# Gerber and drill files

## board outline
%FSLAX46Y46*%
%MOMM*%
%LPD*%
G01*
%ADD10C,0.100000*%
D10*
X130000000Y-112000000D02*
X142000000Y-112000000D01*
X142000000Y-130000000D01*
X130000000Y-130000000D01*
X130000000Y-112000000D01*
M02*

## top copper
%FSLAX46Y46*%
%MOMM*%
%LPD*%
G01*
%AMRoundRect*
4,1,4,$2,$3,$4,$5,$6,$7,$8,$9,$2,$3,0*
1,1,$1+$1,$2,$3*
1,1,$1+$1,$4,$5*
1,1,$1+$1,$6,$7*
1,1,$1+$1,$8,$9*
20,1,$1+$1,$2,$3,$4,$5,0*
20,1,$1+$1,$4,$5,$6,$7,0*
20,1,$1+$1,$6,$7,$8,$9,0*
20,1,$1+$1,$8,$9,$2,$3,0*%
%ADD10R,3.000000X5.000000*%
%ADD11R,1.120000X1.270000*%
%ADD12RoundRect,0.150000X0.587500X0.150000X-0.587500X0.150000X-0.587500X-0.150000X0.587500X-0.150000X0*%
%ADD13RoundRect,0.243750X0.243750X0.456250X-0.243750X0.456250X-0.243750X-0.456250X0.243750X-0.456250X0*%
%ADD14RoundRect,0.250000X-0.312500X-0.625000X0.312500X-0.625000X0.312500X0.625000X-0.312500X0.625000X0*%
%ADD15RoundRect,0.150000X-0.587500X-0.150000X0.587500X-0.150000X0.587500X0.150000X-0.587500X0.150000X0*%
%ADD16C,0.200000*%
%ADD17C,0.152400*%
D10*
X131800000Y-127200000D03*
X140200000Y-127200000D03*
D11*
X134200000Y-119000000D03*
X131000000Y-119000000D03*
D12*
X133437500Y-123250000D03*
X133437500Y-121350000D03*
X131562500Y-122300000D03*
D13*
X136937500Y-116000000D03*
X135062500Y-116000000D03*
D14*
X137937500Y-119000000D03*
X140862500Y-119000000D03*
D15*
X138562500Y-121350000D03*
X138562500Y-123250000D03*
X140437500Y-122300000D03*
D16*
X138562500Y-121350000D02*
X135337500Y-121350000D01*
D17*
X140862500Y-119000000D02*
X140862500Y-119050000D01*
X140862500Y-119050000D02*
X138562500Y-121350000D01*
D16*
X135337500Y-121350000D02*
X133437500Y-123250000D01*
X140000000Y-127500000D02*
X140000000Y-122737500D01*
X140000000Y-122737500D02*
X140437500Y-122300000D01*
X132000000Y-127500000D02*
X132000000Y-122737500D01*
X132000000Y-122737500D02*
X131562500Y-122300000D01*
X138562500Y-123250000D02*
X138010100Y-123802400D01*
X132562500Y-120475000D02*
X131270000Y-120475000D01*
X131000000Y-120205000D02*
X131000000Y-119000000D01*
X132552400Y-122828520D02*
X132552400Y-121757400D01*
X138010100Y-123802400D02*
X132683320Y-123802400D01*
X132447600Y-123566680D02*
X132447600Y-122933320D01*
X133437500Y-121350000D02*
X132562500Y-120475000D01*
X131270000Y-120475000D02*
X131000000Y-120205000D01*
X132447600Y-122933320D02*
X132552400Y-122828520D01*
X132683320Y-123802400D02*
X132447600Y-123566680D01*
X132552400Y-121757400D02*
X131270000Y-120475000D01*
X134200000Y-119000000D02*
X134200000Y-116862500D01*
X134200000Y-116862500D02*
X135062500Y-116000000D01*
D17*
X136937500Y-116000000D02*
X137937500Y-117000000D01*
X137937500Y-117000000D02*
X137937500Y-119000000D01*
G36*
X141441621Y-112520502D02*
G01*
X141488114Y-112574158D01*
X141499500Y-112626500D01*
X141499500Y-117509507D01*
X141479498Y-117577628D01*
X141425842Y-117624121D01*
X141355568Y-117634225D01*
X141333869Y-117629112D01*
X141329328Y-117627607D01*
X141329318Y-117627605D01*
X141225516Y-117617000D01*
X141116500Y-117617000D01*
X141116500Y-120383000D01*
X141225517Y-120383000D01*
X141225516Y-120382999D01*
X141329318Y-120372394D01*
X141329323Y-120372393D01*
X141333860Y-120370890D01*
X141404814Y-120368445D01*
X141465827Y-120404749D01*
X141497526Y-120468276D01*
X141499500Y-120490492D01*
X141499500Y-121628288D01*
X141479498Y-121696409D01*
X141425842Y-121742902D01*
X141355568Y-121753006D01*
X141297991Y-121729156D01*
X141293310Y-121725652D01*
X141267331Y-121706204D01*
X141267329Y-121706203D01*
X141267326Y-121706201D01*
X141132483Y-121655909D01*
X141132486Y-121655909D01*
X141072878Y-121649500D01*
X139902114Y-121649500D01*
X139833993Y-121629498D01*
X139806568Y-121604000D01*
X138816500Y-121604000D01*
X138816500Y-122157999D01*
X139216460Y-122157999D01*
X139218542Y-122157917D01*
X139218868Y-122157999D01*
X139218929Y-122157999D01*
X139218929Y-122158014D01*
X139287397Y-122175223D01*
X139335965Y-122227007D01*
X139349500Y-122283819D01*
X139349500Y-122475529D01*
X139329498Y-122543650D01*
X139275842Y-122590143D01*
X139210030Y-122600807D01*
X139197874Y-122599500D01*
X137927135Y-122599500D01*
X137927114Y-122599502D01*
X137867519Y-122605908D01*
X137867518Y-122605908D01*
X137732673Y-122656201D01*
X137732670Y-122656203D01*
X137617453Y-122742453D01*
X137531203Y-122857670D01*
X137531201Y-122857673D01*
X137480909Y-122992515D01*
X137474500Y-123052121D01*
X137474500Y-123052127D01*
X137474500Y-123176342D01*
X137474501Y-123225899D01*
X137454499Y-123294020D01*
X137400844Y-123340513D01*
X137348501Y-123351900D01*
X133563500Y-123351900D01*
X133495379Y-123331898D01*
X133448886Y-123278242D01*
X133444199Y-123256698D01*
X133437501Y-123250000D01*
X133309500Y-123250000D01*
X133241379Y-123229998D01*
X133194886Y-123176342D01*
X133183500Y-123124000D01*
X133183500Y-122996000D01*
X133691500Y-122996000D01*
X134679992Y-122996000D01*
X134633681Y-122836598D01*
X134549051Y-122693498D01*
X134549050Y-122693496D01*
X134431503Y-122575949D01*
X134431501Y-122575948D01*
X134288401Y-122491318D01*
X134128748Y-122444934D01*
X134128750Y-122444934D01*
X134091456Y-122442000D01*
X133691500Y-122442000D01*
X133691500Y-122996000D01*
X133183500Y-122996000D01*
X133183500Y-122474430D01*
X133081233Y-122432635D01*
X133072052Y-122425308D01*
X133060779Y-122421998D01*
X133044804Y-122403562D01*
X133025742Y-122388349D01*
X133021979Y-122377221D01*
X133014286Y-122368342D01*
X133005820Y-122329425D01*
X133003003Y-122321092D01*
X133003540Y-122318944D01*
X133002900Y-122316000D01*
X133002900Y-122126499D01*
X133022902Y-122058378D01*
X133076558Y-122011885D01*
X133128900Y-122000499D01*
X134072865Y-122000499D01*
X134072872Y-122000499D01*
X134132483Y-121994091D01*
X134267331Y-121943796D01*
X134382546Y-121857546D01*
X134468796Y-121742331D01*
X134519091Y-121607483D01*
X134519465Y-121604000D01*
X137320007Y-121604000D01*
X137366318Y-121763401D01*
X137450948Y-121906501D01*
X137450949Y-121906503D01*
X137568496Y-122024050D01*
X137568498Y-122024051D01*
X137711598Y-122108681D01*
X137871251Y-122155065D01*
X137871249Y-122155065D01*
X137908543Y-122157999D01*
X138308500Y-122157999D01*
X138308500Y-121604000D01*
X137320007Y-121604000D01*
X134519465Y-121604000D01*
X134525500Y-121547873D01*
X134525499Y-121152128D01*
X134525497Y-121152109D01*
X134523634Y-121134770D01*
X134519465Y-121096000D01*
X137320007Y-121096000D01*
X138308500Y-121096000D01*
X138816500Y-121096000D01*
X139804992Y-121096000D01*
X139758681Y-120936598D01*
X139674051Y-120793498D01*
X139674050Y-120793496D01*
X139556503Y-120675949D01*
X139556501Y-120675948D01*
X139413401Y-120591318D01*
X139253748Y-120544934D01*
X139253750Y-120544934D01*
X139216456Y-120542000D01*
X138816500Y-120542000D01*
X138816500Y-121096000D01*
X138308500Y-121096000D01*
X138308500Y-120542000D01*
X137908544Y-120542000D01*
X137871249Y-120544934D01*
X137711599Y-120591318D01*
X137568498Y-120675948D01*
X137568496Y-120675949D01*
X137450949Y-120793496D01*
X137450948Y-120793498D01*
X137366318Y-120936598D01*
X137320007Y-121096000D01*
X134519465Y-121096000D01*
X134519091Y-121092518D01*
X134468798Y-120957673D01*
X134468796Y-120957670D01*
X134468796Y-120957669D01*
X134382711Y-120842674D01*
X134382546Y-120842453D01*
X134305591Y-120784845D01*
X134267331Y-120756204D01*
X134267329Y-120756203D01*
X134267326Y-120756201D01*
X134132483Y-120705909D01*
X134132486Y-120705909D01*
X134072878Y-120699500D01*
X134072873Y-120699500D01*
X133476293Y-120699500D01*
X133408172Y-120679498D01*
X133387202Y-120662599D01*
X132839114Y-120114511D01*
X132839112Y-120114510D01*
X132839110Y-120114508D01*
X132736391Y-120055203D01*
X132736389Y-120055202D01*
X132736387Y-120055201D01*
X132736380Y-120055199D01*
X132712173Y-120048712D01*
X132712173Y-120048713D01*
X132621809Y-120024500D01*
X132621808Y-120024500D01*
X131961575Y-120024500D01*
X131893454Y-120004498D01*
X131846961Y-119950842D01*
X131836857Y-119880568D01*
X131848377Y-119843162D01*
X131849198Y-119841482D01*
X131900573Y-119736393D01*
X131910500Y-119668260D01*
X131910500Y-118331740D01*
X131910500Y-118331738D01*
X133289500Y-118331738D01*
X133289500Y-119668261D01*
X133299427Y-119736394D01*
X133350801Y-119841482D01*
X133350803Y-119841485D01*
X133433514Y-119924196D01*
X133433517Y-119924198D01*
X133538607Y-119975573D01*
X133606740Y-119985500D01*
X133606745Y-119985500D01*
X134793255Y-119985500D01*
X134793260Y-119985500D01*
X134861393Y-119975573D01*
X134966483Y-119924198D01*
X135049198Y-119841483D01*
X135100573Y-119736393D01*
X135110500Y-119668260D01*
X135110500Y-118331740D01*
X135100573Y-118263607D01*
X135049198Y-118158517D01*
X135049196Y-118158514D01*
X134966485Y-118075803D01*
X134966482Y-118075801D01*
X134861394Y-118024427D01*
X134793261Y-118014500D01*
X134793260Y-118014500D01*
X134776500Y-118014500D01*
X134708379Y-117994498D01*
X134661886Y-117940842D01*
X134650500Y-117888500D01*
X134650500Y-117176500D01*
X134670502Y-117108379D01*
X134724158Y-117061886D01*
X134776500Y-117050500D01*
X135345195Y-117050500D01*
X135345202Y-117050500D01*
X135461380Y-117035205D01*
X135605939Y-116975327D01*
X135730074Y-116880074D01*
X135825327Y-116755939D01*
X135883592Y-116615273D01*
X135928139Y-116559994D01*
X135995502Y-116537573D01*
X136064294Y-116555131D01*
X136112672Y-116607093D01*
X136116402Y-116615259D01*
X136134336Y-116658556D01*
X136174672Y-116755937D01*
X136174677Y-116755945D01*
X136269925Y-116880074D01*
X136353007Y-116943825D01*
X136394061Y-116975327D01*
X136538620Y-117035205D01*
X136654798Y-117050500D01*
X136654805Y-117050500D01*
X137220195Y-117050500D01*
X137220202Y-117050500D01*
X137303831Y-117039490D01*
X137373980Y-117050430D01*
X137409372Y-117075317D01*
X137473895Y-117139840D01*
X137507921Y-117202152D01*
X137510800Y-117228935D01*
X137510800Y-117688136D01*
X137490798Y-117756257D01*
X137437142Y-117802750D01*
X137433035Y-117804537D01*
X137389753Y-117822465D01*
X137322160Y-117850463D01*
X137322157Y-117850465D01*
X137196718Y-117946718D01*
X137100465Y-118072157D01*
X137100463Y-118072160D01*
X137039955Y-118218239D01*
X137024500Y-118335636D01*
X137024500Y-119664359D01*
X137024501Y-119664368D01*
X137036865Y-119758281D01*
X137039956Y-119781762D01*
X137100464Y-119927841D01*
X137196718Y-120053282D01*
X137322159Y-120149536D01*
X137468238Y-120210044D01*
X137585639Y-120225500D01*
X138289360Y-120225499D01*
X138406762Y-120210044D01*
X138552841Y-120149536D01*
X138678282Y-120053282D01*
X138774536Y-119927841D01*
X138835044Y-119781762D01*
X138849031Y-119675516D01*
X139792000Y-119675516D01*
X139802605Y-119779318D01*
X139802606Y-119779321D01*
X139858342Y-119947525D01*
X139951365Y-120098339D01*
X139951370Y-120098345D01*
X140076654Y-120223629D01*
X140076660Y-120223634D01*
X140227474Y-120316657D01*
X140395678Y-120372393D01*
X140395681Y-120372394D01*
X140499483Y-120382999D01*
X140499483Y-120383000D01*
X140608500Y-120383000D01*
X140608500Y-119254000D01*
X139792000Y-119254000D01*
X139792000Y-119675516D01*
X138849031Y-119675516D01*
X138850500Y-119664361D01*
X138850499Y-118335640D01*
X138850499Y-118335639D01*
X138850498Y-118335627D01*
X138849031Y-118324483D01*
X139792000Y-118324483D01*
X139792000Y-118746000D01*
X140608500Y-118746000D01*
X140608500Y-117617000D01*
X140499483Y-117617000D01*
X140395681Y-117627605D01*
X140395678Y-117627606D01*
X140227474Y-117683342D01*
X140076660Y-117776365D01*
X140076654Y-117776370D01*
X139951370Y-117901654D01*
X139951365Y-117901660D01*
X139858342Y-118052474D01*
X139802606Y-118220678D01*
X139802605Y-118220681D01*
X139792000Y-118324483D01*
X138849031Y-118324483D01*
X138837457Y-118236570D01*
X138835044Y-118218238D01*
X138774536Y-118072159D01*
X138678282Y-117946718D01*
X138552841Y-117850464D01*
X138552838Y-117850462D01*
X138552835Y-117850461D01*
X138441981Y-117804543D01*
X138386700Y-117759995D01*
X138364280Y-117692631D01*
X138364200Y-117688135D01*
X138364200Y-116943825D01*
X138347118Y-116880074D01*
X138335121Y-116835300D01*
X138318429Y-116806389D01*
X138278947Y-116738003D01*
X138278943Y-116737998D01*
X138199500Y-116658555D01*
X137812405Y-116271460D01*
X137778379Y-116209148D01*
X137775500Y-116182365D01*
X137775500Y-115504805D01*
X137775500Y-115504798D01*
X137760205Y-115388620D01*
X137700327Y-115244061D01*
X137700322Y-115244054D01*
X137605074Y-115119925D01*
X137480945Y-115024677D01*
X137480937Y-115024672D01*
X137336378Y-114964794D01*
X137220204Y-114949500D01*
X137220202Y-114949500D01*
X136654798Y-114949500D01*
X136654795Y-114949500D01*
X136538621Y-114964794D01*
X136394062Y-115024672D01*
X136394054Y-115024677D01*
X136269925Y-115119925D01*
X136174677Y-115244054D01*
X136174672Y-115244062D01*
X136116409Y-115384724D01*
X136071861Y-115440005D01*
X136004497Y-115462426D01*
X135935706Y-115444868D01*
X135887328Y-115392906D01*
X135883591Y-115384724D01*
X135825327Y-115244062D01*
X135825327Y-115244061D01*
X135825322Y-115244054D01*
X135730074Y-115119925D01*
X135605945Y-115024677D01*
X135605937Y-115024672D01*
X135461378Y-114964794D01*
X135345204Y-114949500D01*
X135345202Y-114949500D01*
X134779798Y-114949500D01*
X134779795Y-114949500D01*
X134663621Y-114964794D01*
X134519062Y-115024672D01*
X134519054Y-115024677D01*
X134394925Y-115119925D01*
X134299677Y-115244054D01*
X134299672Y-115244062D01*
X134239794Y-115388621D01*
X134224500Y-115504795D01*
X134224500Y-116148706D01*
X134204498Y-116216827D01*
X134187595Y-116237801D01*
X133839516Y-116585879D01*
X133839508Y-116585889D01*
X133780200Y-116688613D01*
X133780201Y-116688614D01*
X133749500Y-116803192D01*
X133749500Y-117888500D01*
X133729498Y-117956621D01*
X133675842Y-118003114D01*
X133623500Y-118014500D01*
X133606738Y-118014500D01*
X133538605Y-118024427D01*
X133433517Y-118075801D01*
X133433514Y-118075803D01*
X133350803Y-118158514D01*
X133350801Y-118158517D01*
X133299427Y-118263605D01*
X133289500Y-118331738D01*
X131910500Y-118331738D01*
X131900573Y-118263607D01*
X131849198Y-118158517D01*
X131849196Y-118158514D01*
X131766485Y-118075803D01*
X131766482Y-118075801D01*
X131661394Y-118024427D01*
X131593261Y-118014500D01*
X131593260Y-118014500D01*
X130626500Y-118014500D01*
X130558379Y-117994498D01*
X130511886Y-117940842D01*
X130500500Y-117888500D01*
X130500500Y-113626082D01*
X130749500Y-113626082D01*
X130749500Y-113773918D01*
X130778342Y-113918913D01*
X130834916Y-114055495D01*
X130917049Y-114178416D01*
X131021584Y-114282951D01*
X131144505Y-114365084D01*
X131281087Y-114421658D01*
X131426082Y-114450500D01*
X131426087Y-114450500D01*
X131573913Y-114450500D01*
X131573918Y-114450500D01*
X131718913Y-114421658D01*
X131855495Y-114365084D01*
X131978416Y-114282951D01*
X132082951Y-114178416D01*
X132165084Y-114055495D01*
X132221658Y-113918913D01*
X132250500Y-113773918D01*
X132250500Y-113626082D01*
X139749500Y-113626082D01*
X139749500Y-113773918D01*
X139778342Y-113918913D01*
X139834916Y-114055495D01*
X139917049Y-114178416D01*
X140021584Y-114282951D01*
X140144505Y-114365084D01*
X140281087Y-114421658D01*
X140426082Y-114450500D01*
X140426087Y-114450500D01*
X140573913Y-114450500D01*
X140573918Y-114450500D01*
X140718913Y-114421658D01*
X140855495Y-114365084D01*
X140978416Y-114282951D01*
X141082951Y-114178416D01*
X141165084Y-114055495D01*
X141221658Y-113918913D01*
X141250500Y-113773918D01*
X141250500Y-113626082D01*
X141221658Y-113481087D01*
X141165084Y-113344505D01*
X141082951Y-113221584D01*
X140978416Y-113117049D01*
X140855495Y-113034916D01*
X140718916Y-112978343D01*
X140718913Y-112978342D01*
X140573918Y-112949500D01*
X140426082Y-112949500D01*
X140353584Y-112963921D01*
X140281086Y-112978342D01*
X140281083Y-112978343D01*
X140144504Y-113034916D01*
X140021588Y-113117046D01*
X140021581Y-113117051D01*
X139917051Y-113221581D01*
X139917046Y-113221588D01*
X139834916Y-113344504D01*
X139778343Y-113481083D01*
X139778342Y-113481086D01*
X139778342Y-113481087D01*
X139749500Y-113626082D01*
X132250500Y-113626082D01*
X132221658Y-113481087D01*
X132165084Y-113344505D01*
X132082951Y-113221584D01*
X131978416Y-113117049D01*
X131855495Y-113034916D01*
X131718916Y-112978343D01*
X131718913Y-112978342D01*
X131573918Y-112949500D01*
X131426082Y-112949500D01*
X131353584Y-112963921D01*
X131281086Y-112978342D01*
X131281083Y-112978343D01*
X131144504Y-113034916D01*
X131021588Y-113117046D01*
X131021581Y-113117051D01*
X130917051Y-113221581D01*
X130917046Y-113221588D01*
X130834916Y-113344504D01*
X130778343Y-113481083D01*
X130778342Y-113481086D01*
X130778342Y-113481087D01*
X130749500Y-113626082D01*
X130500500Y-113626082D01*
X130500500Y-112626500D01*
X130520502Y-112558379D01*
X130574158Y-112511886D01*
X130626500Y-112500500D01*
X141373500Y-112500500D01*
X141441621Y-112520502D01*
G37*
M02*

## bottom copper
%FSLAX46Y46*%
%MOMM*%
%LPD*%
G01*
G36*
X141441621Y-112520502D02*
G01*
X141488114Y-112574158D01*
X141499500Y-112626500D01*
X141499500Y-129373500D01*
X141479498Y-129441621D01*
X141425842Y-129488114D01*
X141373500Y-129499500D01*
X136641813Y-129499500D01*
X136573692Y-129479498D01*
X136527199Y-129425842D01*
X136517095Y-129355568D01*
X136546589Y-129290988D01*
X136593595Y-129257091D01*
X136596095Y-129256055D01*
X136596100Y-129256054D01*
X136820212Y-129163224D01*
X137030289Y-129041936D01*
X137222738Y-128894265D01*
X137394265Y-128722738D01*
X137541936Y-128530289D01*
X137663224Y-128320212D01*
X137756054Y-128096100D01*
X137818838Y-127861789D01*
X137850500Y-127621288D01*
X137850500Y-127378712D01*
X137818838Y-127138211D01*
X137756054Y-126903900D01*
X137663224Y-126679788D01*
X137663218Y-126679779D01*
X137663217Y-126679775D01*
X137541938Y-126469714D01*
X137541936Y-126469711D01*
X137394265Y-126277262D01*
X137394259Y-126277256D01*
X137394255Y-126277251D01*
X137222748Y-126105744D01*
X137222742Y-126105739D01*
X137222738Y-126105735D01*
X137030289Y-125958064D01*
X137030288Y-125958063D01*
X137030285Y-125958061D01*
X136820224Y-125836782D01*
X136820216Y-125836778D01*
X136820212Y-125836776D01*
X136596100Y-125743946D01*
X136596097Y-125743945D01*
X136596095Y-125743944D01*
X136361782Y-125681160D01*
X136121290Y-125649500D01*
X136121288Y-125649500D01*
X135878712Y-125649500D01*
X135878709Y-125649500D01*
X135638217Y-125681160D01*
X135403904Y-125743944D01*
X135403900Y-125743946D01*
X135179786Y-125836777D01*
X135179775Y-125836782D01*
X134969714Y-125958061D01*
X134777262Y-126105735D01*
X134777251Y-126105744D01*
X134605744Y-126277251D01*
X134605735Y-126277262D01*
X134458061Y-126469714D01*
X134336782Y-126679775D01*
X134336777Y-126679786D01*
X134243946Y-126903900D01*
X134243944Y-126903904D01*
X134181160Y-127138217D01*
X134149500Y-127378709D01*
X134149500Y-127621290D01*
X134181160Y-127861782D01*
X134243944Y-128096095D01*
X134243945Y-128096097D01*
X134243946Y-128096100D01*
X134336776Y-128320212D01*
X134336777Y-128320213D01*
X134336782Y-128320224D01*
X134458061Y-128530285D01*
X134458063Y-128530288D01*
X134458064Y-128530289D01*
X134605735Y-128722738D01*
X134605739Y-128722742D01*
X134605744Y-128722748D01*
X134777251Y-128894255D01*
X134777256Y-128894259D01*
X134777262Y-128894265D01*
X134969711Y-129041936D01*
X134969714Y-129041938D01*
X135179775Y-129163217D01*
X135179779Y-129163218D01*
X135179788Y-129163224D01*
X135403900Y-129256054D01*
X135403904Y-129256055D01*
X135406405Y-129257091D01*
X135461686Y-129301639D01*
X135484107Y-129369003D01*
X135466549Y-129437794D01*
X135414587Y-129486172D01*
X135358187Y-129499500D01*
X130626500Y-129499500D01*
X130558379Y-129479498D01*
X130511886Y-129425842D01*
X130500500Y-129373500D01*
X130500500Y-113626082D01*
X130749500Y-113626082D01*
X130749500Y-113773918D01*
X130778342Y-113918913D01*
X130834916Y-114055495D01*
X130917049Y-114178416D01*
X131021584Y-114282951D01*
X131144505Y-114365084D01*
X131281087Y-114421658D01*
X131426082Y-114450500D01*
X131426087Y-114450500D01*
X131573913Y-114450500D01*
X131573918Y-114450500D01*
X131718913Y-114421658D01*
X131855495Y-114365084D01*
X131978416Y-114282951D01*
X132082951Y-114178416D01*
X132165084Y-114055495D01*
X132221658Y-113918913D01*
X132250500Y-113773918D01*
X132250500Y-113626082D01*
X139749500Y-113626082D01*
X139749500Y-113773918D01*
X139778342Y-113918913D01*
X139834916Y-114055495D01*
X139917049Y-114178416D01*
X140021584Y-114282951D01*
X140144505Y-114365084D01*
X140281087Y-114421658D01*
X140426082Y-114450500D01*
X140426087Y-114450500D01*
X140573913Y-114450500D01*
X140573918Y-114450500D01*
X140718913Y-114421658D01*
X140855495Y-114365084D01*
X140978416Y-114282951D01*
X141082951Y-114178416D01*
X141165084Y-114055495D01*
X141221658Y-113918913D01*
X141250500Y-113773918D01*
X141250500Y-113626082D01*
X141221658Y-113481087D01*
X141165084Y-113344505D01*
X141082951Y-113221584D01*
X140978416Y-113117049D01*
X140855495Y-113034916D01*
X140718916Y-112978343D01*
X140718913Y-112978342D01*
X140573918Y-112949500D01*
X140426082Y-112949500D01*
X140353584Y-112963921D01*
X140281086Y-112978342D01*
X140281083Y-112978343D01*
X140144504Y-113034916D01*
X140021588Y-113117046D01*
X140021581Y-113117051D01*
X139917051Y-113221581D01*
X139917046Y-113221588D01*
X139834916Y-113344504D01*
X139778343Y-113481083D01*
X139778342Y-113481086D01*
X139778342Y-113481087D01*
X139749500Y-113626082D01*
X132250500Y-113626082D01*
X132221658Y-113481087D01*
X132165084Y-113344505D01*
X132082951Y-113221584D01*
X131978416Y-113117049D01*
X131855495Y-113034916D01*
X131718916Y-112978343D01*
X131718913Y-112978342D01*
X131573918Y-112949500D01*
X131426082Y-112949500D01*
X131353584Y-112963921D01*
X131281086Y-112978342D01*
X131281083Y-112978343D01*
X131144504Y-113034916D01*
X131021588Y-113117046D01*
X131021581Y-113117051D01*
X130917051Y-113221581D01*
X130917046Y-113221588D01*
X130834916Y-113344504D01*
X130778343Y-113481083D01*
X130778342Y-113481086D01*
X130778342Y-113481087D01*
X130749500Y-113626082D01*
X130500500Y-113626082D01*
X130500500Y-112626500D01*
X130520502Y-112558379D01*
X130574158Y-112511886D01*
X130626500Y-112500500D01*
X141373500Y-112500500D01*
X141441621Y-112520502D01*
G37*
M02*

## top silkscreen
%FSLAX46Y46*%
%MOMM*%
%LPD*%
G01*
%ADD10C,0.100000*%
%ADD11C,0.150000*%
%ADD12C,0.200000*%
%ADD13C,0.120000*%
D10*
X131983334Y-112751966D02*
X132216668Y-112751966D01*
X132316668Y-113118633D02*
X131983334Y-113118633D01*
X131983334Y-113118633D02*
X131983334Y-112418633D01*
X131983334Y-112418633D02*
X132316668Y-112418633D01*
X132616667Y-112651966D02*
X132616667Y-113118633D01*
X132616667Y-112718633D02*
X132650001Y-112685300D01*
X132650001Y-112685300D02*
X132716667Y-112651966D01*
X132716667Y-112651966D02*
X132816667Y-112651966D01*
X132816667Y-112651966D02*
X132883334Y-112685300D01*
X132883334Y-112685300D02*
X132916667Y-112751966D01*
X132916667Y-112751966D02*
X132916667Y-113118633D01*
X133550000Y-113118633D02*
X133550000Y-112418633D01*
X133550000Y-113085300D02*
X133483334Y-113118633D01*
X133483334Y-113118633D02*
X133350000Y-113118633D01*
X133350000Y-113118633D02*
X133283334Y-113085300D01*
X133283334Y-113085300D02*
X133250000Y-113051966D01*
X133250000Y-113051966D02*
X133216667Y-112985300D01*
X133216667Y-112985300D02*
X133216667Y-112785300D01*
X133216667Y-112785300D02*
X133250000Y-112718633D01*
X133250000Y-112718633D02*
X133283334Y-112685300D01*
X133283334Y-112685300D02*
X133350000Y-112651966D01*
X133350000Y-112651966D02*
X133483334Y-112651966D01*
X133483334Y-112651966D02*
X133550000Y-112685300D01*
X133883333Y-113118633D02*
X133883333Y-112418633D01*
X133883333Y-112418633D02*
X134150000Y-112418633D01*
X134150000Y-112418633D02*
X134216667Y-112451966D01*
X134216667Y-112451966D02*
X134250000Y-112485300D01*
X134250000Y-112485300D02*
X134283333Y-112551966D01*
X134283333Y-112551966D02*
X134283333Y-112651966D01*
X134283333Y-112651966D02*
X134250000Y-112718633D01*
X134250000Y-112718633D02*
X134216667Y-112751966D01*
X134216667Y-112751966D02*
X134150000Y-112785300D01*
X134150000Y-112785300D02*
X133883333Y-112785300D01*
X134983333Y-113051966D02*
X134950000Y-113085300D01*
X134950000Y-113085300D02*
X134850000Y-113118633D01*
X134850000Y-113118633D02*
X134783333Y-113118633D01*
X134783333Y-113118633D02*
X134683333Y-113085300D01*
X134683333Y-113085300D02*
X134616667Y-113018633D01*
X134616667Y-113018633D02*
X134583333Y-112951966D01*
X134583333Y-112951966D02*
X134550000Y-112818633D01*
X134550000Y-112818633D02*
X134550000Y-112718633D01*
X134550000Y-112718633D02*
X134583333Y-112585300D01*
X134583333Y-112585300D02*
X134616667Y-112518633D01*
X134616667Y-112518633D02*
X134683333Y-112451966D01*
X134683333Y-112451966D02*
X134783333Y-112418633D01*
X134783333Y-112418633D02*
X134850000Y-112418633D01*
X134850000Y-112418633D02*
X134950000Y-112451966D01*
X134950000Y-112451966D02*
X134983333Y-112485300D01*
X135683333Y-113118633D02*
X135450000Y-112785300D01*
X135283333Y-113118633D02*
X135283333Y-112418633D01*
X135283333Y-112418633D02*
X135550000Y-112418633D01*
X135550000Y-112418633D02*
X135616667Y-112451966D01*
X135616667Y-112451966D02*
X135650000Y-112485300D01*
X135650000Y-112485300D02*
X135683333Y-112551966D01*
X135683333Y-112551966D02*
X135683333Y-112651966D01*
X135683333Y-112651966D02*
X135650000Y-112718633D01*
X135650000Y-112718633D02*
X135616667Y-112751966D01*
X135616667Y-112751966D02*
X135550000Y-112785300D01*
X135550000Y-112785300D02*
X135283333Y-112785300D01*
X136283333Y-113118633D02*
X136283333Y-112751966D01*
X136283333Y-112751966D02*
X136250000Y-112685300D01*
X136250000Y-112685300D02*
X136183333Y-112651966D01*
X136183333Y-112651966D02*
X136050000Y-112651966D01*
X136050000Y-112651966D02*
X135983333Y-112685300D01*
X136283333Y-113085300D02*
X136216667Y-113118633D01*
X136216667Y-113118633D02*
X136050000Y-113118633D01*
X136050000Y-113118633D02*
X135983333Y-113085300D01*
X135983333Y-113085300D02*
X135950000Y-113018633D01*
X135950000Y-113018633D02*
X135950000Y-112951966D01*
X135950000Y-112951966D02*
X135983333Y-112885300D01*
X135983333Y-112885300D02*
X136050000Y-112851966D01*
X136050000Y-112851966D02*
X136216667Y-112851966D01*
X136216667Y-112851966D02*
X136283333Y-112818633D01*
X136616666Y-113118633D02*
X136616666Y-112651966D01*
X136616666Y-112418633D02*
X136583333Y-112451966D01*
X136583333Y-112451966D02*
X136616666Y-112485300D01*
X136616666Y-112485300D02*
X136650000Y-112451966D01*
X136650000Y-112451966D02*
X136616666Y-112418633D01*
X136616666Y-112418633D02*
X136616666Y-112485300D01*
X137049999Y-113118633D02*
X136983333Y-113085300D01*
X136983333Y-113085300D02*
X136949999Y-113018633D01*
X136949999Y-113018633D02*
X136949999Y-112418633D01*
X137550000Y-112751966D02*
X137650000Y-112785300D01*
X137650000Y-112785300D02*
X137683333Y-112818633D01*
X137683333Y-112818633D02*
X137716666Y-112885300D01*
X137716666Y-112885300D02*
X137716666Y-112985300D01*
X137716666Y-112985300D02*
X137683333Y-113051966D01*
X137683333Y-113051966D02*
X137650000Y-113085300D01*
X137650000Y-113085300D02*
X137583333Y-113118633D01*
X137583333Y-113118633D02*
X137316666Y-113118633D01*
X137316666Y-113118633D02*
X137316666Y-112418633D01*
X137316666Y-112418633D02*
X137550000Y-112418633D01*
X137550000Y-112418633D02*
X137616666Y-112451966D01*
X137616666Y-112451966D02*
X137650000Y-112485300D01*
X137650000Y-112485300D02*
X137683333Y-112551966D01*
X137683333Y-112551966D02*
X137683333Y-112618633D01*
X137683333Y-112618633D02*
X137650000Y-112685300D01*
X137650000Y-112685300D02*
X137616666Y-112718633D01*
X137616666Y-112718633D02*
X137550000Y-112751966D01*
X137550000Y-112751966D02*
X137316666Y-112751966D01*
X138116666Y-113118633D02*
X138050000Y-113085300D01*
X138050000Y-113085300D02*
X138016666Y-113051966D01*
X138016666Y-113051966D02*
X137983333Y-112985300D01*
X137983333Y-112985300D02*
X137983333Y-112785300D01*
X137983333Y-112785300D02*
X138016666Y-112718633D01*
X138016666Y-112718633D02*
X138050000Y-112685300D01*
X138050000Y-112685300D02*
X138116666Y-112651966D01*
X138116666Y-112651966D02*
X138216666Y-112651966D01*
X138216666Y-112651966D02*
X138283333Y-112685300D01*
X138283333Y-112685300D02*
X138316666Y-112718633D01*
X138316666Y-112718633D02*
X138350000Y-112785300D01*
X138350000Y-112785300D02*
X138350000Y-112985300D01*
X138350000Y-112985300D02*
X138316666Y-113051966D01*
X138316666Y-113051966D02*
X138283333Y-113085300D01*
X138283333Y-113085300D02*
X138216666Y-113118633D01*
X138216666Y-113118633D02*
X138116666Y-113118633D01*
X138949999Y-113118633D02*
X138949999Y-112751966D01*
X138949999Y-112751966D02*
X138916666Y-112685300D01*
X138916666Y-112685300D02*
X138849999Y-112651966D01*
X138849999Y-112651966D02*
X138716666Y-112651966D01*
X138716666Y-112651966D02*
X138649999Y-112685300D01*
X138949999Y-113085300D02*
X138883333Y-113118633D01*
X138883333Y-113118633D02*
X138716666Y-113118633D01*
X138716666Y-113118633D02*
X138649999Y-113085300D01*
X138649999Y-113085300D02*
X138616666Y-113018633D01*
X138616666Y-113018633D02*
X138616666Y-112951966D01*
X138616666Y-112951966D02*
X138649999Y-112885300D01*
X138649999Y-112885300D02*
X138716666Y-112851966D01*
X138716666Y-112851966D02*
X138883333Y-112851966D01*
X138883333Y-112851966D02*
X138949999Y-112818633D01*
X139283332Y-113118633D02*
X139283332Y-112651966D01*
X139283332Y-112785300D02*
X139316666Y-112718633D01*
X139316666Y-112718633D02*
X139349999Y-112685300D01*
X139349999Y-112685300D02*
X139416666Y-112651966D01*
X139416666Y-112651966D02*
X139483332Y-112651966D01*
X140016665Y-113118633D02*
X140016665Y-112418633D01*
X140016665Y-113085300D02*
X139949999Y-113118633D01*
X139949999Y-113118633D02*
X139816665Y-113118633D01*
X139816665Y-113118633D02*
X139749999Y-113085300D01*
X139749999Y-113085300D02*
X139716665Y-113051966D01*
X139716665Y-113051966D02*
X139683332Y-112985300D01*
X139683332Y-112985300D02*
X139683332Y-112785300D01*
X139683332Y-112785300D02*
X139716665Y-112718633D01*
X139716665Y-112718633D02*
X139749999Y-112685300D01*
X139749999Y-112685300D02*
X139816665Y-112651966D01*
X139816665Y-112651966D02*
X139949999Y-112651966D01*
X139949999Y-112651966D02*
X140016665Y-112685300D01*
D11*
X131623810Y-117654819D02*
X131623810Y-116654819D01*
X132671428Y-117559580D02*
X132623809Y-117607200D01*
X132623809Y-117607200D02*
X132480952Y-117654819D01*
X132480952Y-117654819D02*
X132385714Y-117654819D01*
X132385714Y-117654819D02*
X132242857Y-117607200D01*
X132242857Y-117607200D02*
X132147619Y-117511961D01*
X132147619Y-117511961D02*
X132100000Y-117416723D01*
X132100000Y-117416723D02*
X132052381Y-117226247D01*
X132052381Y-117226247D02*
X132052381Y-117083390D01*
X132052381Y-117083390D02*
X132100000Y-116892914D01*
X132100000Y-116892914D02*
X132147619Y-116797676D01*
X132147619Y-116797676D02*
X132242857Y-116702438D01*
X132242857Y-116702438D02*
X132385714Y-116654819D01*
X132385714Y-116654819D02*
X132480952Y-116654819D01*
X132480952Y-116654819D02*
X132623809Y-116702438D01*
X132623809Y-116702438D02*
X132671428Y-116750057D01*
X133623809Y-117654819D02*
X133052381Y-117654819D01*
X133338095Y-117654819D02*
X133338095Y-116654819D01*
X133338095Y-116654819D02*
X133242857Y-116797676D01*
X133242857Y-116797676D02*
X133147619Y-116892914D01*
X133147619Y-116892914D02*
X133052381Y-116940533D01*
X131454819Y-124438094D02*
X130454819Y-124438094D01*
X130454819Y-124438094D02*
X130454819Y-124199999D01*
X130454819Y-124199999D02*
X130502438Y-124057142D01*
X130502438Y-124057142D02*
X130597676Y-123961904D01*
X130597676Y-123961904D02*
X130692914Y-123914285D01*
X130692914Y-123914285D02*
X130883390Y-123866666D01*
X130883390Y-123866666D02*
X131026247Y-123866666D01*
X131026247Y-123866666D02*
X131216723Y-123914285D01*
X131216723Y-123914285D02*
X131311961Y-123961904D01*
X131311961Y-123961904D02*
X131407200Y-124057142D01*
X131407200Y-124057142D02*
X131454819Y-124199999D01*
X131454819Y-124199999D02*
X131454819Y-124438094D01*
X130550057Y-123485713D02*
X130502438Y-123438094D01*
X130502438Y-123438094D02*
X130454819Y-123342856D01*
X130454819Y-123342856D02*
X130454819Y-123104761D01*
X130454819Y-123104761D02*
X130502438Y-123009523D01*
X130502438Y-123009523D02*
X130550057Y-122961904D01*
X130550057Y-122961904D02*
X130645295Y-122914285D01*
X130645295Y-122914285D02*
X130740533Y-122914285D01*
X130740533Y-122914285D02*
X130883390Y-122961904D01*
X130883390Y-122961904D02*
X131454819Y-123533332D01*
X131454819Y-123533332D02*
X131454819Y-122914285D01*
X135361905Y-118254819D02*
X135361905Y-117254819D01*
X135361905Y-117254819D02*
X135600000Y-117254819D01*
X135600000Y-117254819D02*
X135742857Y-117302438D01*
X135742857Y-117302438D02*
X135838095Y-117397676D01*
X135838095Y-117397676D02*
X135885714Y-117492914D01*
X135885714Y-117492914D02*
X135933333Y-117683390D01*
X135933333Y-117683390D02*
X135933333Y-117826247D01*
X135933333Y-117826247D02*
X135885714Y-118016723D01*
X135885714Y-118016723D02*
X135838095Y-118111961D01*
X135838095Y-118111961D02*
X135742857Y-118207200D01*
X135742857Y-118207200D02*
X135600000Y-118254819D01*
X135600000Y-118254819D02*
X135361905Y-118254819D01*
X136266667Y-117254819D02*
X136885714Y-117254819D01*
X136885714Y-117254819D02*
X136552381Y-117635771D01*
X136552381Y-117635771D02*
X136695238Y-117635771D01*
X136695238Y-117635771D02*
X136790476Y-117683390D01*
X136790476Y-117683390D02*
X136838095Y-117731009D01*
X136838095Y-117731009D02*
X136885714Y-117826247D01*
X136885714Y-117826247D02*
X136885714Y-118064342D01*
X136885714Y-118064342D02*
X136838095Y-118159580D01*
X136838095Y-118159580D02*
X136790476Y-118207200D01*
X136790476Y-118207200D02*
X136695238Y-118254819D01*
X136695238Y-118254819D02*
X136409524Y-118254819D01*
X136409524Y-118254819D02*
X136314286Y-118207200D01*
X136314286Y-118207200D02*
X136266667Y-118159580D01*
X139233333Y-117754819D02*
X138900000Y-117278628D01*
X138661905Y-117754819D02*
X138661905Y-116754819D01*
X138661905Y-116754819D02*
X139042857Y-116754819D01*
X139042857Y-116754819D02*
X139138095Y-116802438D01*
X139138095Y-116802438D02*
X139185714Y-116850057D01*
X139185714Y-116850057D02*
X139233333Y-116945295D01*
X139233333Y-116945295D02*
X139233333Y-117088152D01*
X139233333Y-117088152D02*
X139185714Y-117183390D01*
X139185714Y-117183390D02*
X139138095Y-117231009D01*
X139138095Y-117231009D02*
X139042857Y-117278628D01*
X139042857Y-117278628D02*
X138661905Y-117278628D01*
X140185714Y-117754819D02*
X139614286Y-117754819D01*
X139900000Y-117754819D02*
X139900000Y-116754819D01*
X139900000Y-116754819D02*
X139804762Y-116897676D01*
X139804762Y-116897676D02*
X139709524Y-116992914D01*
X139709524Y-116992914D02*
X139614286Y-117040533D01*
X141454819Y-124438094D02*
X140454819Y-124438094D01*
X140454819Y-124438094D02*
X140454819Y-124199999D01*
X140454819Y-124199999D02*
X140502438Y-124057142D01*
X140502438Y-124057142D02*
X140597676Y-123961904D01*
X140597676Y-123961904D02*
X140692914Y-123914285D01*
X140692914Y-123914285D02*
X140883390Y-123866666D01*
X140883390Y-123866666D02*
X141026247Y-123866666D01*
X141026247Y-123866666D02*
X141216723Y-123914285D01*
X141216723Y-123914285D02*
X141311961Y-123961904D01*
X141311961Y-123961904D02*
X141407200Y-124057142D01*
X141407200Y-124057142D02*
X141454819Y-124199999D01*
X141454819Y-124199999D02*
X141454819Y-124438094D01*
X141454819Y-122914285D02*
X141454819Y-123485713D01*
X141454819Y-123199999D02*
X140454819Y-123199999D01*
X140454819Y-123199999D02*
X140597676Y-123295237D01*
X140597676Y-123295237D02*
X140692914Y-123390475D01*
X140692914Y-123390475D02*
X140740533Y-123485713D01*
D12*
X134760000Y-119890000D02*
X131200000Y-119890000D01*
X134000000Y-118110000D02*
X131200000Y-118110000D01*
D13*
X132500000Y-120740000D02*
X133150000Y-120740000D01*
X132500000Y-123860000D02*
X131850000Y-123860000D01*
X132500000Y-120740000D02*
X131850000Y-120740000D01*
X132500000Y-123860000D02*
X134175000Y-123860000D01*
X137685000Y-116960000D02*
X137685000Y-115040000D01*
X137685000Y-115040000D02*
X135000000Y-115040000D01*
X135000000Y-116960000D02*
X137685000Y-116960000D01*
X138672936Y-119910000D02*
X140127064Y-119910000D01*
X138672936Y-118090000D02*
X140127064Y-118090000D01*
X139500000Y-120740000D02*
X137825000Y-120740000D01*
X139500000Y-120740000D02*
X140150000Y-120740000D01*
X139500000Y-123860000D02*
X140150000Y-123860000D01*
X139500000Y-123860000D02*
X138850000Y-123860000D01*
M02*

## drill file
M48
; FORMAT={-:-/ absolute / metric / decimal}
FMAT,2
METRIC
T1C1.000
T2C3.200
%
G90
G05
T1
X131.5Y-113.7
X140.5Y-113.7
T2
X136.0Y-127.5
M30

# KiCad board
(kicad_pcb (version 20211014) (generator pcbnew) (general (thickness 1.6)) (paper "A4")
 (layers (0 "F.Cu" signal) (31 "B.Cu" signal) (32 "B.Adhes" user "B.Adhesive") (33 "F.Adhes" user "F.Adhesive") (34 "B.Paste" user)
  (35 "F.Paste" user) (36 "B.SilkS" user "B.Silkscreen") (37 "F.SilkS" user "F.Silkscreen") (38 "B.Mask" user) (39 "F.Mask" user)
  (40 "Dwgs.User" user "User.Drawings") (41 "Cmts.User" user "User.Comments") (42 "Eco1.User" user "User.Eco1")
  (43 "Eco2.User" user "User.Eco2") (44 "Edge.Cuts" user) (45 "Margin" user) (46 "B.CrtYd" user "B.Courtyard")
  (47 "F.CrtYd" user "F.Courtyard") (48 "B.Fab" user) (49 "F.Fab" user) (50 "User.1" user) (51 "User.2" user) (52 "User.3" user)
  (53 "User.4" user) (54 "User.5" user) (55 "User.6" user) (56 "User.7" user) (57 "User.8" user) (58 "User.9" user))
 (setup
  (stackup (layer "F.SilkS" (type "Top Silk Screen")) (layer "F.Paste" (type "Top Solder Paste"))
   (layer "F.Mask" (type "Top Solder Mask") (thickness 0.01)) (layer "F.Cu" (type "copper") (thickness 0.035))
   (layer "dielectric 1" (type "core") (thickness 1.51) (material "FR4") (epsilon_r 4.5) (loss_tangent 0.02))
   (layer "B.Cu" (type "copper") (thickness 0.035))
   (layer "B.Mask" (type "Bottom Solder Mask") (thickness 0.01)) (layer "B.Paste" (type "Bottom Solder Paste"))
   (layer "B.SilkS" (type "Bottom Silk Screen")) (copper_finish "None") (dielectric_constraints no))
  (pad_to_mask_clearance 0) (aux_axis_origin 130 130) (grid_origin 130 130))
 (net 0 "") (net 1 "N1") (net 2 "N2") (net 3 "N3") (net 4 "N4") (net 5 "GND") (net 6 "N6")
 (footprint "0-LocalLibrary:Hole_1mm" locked (layer "F.Cu") (at 131.5 113.7)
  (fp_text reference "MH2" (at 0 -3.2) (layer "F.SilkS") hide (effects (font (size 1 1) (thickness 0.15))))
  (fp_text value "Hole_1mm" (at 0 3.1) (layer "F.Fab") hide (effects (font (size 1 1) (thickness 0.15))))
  (pad "" np_thru_hole circle locked (at 0 0) (size 1 1) (drill 1) (layers F&B.Cu *.Mask)))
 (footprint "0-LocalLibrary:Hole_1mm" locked (layer "F.Cu") (at 140.5 113.7)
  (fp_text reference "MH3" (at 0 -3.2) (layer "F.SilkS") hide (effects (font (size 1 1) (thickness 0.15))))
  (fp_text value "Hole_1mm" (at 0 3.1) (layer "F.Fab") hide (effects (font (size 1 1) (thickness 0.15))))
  (pad "" np_thru_hole circle locked (at 0 0) (size 1 1) (drill 1) (layers F&B.Cu *.Mask)))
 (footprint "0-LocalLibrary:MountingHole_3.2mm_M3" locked (layer "F.Cu") (at 136 127.5)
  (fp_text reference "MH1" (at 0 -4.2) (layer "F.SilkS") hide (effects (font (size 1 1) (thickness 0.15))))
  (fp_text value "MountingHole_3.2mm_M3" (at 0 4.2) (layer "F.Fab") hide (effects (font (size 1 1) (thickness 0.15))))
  (pad "" np_thru_hole circle locked (at 0 0) (size 3.2 3.2) (drill 3.2) (layers *.Cu *.Mask)))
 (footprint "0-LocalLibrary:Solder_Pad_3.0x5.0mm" (layer "F.Cu") (at 131.8 127.2)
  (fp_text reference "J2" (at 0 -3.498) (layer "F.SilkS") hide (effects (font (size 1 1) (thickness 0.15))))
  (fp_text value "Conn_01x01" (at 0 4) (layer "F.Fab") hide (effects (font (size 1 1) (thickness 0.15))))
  (pad "1" smd rect (at 0 0) (size 3 5) (layers "F.Cu" "F.Mask") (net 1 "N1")))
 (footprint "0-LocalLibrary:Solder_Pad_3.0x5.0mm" (layer "F.Cu") (at 140.2 127.2)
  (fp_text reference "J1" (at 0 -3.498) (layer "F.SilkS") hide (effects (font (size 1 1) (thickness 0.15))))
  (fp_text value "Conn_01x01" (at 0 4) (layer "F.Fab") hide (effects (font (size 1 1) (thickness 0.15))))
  (pad "1" smd rect (at 0 0) (size 3 5) (layers "F.Cu" "F.Mask") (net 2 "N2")))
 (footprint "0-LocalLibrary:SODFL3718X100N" (layer "F.Cu") (at 132.6 119 180)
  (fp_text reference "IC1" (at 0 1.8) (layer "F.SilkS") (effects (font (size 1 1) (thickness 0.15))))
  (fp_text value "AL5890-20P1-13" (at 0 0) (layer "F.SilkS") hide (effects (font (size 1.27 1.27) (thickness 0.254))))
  (fp_line (start -2.16 -0.89) (end 1.4 -0.89) (layer "F.SilkS") (width 0.2))
  (fp_line (start -1.4 0.89) (end 1.4 0.89) (layer "F.SilkS") (width 0.2))
  (pad "1" smd rect (at -1.6 0 180) (size 1.12 1.27) (layers "F.Cu" "F.Paste" "F.Mask") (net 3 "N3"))
  (pad "2" smd rect (at 1.6 0 180) (size 1.12 1.27) (layers "F.Cu" "F.Paste" "F.Mask") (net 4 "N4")))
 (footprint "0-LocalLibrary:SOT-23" (layer "F.Cu") (at 132.5 122.3 180)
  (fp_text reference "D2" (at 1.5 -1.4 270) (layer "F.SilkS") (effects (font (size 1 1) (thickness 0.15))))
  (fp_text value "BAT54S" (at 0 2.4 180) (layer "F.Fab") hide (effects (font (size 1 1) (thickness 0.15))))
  (fp_line (start 0 1.56) (end -0.65 1.56) (layer "F.SilkS") (width 0.12))
  (fp_line (start 0 -1.56) (end 0.65 -1.56) (layer "F.SilkS") (width 0.12))
  (fp_line (start 0 1.56) (end 0.65 1.56) (layer "F.SilkS") (width 0.12))
  (fp_line (start 0 -1.56) (end -1.675 -1.56) (layer "F.SilkS") (width 0.12))
  (pad "1" smd roundrect (at -0.9375 -0.95 180) (size 1.475 0.6) (layers "F.Cu" "F.Paste" "F.Mask") (roundrect_rratio 0.25) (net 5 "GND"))
  (pad "2" smd roundrect (at -0.9375 0.95 180) (size 1.475 0.6) (layers "F.Cu" "F.Paste" "F.Mask") (roundrect_rratio 0.25) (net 4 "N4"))
  (pad "3" smd roundrect (at 0.9375 0 180) (size 1.475 0.6) (layers "F.Cu" "F.Paste" "F.Mask") (roundrect_rratio 0.25) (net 1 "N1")))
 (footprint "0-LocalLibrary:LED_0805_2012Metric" (layer "F.Cu") (at 136 116 180)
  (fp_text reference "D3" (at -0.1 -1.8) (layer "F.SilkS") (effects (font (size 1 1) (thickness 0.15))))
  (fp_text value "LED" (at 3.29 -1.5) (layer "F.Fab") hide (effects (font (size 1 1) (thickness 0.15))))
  (fp_line (start -1.685 -0.96) (end -1.685 0.96) (layer "F.SilkS") (width 0.12))
  (fp_line (start -1.685 0.96) (end 1 0.96) (layer "F.SilkS") (width 0.12))
  (fp_line (start 1 -0.96) (end -1.685 -0.96) (layer "F.SilkS") (width 0.12))
  (pad "1" smd roundrect (at -0.9375 0 180) (size 0.975 1.4) (layers "F.Cu" "F.Paste" "F.Mask") (roundrect_rratio 0.25) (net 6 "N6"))
  (pad "2" smd roundrect (at 0.9375 0 180) (size 0.975 1.4) (layers "F.Cu" "F.Paste" "F.Mask") (roundrect_rratio 0.25) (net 3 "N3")))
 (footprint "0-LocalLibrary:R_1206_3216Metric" (layer "F.Cu") (at 139.4 119) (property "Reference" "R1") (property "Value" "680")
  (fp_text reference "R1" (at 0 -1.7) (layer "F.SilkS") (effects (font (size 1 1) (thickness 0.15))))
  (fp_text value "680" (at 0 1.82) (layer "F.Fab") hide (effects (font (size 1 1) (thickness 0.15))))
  (fp_line (start -0.727064 0.91) (end 0.727064 0.91) (layer "F.SilkS") (width 0.12))
  (fp_line (start -0.727064 -0.91) (end 0.727064 -0.91) (layer "F.SilkS") (width 0.12))
  (pad "1" smd roundrect (at -1.4625 0) (size 1.125 1.75) (layers "F.Cu" "F.Paste" "F.Mask") (roundrect_rratio 0.222222) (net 6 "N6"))
  (pad "2" smd roundrect (at 1.4625 0) (size 1.125 1.75) (layers "F.Cu" "F.Paste" "F.Mask") (roundrect_rratio 0.222222) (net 5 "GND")))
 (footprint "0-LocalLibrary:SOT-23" (layer "F.Cu") (at 139.5 122.3)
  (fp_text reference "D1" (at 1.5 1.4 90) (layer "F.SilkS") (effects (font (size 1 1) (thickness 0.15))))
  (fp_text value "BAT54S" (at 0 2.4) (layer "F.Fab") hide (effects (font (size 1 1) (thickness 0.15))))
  (fp_line (start 0 -1.56) (end -1.675 -1.56) (layer "F.SilkS") (width 0.12))
  (fp_line (start 0 -1.56) (end 0.65 -1.56) (layer "F.SilkS") (width 0.12))
  (fp_line (start 0 1.56) (end 0.65 1.56) (layer "F.SilkS") (width 0.12))
  (fp_line (start 0 1.56) (end -0.65 1.56) (layer "F.SilkS") (width 0.12))
  (pad "1" smd roundrect (at -0.9375 -0.95) (size 1.475 0.6) (layers "F.Cu" "F.Paste" "F.Mask") (roundrect_rratio 0.25) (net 5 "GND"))
  (pad "2" smd roundrect (at -0.9375 0.95) (size 1.475 0.6) (layers "F.Cu" "F.Paste" "F.Mask") (roundrect_rratio 0.25) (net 4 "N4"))
  (pad "3" smd roundrect (at 0.9375 0) (size 1.475 0.6) (layers "F.Cu" "F.Paste" "F.Mask") (roundrect_rratio 0.25) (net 2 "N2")))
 (gr_rect (start 130 130) (end 142 112) (layer "Edge.Cuts") (width 0.1) (fill none))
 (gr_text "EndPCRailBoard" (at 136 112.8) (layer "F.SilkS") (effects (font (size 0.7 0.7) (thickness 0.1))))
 (segment (start 138.5625 121.35) (end 135.3375 121.35) (width 0.2) (layer "F.Cu") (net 5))
 (segment (start 140.8625 119) (end 140.8625 119.05) (width 0.1524) (layer "F.Cu") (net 5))
 (segment (start 140.8625 119.05) (end 138.5625 121.35) (width 0.1524) (layer "F.Cu") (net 5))
 (segment (start 135.3375 121.35) (end 133.4375 123.25) (width 0.2) (layer "F.Cu") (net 5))
 (segment (start 140 127.5) (end 140 122.7375) (width 0.2) (layer "F.Cu") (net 2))
 (segment (start 140 122.7375) (end 140.4375 122.3) (width 0.2) (layer "F.Cu") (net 2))
 (segment (start 132 127.5) (end 132 122.7375) (width 0.2) (layer "F.Cu") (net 1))
 (segment (start 132 122.7375) (end 131.5625 122.3) (width 0.2) (layer "F.Cu") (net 1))
 (segment (start 138.5625 123.25) (end 138.0101 123.8024) (width 0.2) (layer "F.Cu") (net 4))
 (segment (start 132.5625 120.475) (end 131.27 120.475) (width 0.2) (layer "F.Cu") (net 4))
 (segment (start 131 120.205) (end 131 119) (width 0.2) (layer "F.Cu") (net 4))
 (segment (start 132.5524 122.82852) (end 132.5524 121.7574) (width 0.2) (layer "F.Cu") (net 4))
 (segment (start 138.0101 123.8024) (end 132.68332 123.8024) (width 0.2) (layer "F.Cu") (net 4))
 (segment (start 132.4476 123.56668) (end 132.4476 122.93332) (width 0.2) (layer "F.Cu") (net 4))
 (segment (start 133.4375 121.35) (end 132.5625 120.475) (width 0.2) (layer "F.Cu") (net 4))
 (segment (start 131.27 120.475) (end 131 120.205) (width 0.2) (layer "F.Cu") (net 4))
 (segment (start 132.4476 122.93332) (end 132.5524 122.82852) (width 0.2) (layer "F.Cu") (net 4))
 (segment (start 132.68332 123.8024) (end 132.4476 123.56668) (width 0.2) (layer "F.Cu") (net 4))
 (segment (start 132.5524 121.7574) (end 131.27 120.475) (width 0.2) (layer "F.Cu") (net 4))
 (segment (start 134.2 119) (end 134.2 116.8625) (width 0.2) (layer "F.Cu") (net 3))
 (segment (start 134.2 116.8625) (end 135.0625 116) (width 0.2) (layer "F.Cu") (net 3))
 (segment (start 136.9375 116) (end 137.9375 117) (width 0.1524) (layer "F.Cu") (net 6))
 (segment (start 137.9375 117) (end 137.9375 119) (width 0.1524) (layer "F.Cu") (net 6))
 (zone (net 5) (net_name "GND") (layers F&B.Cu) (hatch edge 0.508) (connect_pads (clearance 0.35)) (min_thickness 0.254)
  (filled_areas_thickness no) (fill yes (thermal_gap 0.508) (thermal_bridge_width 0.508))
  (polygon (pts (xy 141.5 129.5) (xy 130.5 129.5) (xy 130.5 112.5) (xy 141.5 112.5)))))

